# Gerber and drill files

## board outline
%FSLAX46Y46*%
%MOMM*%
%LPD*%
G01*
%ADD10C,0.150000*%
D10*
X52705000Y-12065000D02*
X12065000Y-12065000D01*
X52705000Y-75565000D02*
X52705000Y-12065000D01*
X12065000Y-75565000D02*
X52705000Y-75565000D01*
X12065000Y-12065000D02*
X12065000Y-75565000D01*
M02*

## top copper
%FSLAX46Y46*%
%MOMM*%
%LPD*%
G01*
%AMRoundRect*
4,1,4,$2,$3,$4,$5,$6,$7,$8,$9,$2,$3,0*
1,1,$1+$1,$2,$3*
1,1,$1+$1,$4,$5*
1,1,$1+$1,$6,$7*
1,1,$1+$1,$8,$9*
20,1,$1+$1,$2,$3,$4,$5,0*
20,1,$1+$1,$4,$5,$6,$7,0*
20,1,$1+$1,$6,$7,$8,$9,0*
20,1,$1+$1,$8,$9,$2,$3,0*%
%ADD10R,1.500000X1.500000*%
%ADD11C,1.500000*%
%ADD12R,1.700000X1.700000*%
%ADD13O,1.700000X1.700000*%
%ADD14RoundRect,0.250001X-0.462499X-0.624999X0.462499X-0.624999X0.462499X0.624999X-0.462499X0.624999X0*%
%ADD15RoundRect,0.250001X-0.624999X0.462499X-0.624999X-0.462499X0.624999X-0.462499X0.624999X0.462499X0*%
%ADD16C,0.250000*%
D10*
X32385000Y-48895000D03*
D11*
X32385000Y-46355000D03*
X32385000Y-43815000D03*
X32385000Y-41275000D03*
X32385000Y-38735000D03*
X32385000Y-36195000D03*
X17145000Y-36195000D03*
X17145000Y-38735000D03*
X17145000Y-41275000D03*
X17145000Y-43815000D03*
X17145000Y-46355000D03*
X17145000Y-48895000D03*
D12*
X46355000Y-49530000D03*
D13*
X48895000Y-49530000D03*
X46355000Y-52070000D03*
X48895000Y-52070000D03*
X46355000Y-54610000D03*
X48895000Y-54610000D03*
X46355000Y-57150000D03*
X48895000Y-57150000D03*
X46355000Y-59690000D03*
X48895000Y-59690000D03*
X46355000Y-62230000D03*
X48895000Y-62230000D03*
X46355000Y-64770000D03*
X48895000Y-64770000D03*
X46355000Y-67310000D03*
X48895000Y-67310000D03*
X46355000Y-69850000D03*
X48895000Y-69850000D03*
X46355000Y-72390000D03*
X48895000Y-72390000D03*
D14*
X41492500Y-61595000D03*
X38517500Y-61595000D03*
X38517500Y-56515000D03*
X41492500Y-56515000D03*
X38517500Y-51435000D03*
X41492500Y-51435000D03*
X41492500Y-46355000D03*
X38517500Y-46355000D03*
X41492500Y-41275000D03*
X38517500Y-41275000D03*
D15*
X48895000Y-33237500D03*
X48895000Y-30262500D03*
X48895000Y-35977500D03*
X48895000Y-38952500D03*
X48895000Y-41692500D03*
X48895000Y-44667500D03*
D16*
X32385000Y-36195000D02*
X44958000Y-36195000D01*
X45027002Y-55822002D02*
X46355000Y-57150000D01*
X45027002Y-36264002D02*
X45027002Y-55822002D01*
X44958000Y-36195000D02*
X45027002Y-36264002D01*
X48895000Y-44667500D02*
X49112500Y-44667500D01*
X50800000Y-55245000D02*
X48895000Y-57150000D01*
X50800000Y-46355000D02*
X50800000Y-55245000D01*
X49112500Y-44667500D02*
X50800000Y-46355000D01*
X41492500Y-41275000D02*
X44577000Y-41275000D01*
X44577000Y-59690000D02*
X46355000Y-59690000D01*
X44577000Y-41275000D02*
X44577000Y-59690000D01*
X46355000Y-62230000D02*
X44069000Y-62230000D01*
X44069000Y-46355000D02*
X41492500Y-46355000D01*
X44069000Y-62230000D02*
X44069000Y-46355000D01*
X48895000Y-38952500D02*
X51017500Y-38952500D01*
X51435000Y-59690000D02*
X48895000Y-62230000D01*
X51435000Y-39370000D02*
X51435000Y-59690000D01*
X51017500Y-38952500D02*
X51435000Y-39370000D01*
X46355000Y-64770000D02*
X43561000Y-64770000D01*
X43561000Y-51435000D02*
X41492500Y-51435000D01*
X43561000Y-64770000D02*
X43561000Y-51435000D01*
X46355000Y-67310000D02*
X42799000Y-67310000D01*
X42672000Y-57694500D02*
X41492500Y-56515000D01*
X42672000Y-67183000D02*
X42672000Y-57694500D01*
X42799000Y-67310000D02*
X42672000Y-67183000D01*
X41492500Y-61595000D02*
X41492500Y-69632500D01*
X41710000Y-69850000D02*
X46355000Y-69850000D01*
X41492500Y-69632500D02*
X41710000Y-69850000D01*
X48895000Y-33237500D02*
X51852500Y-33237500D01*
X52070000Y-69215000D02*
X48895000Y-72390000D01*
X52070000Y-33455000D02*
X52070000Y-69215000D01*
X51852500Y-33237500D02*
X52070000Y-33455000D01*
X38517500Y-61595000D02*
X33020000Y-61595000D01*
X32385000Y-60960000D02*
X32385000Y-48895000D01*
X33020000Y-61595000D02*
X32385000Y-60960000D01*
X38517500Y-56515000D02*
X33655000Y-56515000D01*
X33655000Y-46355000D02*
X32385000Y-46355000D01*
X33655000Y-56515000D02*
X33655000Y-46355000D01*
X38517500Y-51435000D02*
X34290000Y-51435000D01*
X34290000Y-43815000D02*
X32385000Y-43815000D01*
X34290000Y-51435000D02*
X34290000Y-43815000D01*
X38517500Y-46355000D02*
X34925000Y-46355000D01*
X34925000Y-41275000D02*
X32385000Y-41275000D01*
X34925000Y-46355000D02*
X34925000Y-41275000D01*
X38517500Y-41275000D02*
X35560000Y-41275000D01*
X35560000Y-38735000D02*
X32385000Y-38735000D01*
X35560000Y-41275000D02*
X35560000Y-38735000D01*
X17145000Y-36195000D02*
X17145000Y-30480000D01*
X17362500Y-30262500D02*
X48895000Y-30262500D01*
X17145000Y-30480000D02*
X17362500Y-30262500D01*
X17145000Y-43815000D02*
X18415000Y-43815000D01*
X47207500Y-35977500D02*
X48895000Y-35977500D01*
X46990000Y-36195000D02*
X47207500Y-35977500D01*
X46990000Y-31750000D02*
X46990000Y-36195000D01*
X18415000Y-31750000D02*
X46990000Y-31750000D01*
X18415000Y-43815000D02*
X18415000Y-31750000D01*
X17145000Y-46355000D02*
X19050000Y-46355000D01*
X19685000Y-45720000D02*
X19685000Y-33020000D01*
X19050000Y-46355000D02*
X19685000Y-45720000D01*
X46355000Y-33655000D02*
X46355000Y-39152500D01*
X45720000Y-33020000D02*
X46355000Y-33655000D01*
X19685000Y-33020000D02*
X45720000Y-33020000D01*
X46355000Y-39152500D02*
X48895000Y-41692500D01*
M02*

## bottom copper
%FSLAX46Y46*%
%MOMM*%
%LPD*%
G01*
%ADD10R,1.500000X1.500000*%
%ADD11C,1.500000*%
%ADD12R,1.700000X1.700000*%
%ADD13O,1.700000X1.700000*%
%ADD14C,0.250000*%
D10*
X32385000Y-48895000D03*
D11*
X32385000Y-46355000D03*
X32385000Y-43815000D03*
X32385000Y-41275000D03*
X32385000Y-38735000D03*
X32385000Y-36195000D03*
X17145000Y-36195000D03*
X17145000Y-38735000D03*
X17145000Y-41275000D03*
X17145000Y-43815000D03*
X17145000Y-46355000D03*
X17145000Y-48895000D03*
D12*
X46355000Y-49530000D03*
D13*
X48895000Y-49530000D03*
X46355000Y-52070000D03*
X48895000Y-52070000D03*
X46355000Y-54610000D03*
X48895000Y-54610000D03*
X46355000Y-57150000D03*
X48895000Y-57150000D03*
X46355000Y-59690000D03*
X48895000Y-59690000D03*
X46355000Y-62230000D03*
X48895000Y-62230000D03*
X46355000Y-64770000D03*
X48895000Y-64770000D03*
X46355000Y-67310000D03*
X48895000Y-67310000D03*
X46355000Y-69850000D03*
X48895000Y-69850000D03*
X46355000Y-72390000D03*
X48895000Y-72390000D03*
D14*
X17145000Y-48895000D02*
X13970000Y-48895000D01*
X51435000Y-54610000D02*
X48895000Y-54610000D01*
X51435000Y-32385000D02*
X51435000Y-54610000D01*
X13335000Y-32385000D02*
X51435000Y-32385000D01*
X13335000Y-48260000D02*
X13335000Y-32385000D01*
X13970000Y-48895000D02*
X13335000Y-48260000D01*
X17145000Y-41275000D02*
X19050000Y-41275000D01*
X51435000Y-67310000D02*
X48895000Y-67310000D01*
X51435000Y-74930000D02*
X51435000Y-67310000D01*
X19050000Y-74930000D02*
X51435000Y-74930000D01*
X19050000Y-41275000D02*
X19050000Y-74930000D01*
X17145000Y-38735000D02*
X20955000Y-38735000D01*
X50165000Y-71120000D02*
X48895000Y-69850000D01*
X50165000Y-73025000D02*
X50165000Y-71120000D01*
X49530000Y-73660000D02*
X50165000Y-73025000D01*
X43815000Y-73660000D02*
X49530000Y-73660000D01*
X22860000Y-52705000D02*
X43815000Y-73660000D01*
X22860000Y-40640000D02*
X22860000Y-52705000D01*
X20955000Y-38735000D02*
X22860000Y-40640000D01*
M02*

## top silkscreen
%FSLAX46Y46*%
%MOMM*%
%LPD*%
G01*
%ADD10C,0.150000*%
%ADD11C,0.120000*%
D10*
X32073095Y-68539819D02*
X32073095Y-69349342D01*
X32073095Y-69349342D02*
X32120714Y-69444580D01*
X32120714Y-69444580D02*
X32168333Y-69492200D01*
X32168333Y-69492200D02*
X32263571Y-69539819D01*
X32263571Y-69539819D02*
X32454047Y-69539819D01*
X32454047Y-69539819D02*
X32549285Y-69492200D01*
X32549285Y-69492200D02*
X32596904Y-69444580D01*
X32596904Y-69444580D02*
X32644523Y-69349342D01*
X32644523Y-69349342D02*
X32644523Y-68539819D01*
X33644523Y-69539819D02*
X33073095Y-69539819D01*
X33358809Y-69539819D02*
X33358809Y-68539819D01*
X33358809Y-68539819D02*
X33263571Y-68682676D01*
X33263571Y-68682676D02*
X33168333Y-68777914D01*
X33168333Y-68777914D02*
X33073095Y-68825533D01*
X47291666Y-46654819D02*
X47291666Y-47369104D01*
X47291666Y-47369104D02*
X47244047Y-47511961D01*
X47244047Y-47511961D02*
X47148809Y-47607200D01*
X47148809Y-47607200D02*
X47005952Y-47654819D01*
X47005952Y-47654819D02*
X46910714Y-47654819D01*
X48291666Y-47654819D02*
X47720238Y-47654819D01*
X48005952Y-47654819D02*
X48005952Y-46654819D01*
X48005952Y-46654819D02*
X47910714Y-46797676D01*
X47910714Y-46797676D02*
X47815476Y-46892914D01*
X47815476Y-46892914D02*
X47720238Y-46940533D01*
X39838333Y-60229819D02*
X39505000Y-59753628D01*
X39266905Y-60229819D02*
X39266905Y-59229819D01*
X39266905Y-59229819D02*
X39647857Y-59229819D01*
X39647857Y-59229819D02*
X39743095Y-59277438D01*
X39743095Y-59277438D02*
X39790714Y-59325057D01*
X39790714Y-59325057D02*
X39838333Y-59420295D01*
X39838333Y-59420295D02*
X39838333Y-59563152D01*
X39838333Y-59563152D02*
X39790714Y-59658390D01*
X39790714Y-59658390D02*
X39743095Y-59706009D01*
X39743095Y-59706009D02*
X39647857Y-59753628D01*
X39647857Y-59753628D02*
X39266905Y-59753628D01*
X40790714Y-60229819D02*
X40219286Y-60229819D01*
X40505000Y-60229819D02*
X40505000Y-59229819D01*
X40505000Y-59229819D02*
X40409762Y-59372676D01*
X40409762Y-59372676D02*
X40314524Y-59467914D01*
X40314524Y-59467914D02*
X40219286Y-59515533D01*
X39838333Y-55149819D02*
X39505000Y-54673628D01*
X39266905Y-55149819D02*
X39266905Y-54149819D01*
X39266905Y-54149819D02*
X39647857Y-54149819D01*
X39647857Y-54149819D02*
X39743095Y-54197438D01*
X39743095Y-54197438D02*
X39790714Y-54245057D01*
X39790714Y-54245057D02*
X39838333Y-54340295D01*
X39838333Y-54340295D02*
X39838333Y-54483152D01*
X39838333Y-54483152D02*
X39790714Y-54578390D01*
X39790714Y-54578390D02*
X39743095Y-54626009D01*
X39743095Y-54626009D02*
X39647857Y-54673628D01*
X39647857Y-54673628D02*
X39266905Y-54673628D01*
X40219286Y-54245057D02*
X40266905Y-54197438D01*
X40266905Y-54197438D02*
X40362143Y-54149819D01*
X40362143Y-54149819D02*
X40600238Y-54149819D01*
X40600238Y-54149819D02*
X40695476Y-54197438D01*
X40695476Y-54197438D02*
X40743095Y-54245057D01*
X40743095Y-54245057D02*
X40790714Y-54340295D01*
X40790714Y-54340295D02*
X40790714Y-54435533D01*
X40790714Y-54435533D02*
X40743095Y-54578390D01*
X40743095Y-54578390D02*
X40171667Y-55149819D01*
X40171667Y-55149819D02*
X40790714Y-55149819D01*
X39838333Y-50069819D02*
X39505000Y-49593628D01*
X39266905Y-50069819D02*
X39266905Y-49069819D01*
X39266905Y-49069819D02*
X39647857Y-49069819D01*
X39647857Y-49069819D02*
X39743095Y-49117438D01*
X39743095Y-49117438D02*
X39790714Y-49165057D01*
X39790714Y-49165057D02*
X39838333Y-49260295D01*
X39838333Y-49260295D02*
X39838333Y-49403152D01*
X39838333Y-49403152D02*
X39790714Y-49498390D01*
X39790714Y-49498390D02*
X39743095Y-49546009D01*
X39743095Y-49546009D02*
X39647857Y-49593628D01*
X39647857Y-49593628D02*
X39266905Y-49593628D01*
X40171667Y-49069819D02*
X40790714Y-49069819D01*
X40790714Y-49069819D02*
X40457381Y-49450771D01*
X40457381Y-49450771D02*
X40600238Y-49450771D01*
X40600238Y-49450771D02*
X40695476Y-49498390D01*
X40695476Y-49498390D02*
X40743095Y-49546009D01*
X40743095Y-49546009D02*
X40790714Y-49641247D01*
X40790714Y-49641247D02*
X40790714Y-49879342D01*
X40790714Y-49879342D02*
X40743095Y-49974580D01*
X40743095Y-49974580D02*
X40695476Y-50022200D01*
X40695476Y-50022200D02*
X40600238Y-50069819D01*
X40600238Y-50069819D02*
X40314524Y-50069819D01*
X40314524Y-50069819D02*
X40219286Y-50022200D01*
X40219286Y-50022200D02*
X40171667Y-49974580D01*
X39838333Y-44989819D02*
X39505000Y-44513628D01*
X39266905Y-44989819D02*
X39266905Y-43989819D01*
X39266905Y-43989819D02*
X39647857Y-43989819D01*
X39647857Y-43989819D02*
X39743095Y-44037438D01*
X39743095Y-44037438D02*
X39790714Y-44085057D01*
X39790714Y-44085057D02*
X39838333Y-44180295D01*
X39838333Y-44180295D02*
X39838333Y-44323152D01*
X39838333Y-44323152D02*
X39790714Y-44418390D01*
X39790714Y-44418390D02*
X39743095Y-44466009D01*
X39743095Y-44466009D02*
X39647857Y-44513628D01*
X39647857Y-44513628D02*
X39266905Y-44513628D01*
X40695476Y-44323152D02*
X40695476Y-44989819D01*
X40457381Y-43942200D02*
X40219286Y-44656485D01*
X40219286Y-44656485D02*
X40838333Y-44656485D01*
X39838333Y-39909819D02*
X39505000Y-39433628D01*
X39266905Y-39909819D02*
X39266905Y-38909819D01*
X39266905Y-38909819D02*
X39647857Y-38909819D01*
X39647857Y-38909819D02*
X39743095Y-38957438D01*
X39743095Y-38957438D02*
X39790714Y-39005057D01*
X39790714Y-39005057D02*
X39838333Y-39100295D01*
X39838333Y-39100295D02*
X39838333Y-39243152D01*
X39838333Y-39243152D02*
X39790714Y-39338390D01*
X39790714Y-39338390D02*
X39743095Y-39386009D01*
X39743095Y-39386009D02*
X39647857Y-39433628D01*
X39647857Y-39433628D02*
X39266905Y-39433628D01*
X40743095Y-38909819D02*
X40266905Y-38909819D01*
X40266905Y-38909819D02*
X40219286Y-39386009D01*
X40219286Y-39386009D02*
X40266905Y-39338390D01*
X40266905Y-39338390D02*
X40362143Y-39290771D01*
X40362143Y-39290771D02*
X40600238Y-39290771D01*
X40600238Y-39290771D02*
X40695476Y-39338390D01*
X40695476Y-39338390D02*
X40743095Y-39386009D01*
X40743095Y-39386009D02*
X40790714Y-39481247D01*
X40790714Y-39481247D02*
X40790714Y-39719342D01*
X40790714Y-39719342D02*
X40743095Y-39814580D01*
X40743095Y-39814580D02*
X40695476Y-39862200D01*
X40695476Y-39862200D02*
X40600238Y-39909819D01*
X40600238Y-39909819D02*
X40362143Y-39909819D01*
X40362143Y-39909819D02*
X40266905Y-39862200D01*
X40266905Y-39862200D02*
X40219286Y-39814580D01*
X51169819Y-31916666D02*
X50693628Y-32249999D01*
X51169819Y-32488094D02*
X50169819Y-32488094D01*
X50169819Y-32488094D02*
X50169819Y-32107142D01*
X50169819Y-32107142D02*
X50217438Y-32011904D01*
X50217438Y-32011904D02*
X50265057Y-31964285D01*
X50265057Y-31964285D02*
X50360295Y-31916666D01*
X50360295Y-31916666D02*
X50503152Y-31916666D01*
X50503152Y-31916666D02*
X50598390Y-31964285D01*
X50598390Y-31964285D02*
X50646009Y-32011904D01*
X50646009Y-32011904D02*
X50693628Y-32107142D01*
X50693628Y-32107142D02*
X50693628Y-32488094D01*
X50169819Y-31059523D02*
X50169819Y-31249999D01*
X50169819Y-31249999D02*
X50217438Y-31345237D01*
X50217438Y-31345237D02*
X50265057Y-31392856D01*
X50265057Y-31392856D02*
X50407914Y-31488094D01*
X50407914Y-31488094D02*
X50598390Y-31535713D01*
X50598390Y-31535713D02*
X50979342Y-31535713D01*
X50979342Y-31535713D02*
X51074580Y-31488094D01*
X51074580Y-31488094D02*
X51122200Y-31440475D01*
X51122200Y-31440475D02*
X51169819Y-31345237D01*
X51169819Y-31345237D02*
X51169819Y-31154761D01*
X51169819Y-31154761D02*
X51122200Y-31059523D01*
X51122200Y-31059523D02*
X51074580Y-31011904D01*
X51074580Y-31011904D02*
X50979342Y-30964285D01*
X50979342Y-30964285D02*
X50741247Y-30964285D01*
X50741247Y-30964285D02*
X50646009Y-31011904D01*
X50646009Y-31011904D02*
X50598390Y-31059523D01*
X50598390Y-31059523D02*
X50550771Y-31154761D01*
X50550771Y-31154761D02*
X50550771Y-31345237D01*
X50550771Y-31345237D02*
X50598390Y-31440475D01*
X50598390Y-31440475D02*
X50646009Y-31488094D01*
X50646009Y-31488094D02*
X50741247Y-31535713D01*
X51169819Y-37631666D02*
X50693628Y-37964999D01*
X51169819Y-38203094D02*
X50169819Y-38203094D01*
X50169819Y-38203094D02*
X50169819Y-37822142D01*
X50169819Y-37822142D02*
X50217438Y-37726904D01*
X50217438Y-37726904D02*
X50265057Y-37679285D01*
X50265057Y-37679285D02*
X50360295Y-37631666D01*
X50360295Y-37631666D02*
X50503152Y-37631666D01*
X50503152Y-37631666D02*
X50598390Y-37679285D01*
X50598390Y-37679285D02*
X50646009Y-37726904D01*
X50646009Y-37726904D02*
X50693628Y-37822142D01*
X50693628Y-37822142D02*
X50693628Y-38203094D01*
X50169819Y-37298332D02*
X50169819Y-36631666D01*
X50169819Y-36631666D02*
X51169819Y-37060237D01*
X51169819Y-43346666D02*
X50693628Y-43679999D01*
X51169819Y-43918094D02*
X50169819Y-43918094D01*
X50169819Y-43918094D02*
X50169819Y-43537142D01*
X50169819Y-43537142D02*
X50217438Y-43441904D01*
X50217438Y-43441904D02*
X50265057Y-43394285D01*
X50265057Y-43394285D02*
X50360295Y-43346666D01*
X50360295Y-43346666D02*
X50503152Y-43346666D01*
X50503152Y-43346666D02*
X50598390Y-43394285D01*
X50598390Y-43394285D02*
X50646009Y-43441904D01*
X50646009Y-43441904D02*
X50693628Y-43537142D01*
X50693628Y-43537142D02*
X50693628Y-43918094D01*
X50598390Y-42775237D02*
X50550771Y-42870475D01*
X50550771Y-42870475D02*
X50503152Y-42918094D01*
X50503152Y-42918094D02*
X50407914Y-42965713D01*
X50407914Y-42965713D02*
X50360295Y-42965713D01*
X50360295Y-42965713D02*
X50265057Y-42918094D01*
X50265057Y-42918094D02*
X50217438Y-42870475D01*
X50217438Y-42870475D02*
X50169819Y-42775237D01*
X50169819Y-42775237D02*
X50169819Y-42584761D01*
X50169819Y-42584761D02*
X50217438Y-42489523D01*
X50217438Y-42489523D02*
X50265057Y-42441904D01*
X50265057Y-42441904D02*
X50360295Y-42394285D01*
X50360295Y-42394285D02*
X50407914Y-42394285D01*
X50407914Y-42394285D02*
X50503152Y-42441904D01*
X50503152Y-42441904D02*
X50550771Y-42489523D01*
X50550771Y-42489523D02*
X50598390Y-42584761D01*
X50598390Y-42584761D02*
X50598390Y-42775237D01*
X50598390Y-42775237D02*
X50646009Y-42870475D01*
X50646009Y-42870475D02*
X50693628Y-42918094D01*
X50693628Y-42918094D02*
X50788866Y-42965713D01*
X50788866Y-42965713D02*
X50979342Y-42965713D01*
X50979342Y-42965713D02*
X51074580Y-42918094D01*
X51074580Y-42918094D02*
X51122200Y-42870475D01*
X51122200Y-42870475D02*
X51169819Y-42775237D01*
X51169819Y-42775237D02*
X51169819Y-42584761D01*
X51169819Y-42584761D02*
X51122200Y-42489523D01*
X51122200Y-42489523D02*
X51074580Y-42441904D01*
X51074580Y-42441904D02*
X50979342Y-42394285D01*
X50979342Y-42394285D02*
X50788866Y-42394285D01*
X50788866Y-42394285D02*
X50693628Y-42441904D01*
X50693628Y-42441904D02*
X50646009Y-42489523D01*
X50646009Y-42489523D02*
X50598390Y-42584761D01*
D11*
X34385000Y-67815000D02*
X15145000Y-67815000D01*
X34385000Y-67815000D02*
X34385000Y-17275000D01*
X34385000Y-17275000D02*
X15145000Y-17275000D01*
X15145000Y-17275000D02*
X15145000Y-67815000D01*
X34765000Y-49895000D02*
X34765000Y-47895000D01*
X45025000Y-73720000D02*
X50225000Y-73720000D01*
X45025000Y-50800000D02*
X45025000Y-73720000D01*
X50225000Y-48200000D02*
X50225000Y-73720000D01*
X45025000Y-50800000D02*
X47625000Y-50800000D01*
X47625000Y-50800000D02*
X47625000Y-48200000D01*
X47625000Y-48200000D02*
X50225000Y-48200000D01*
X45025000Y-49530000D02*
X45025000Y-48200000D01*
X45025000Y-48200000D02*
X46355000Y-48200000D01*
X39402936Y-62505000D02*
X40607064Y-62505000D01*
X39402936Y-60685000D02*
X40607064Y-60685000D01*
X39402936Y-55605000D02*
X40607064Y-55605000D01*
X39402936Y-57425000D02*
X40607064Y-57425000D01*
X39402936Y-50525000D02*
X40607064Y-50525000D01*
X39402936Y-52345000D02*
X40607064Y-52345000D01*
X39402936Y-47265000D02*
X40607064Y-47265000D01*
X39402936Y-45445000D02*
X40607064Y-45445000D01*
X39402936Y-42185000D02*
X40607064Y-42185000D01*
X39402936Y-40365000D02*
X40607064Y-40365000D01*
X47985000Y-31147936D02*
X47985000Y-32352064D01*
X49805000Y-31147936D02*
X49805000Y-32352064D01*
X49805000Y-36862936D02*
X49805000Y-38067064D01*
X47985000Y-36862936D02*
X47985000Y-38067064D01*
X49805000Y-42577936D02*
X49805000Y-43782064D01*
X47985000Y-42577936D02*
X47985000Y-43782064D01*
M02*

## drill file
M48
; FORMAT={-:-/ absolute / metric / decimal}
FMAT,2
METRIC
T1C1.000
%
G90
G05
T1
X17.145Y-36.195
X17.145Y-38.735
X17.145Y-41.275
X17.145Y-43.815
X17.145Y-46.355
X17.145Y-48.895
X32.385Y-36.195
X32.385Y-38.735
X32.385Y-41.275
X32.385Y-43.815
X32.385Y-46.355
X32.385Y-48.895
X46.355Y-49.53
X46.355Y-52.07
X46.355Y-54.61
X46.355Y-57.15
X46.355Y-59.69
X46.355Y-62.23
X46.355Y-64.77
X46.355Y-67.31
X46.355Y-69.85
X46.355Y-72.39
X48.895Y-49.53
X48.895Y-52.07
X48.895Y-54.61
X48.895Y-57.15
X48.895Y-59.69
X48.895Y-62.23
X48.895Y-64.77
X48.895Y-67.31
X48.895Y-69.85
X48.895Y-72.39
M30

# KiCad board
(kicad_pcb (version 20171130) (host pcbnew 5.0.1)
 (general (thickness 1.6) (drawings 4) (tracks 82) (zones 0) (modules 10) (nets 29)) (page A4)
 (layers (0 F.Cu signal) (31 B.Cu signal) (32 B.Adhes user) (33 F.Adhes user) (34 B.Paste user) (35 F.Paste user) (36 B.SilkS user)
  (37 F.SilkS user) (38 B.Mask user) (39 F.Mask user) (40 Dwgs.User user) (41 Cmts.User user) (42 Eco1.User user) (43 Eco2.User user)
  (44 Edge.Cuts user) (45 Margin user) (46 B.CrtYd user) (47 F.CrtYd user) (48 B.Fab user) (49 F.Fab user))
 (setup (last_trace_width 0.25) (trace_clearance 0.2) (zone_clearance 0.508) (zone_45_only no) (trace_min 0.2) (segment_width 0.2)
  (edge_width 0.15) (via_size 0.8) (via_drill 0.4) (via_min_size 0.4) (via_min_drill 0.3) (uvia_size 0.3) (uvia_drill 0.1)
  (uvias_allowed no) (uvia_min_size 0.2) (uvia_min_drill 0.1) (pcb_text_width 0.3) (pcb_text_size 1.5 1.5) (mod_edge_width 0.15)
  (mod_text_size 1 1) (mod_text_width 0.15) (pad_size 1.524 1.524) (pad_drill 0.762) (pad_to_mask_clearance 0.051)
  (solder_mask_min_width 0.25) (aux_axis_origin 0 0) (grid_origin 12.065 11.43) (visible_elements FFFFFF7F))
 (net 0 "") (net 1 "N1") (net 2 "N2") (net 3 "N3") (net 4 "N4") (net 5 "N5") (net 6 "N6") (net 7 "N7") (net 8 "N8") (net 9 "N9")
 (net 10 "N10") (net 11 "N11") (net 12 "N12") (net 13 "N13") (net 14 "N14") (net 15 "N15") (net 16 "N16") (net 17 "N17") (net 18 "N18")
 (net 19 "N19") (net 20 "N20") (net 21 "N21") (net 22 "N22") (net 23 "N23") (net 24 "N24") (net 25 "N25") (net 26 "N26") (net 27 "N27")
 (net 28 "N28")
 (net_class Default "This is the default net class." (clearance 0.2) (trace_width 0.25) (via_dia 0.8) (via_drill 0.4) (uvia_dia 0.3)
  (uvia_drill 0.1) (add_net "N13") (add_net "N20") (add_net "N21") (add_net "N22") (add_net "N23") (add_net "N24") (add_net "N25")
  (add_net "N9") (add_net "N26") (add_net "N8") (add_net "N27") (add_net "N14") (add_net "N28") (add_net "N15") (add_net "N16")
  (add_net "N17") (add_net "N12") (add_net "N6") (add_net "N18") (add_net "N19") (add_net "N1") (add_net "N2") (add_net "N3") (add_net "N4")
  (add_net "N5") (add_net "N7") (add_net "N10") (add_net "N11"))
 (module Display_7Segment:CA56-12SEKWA (layer F.Cu) (at 32.385 48.895 180)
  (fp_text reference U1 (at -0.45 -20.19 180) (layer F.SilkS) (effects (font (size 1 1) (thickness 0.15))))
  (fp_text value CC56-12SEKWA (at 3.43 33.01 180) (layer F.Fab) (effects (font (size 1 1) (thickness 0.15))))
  (fp_line (start -2 -18.92) (end 17.24 -18.92) (layer F.SilkS) (width 0.12))
  (fp_line (start -2 -18.92) (end -2 31.62) (layer F.SilkS) (width 0.12))
  (fp_line (start -2 31.62) (end 17.24 31.62) (layer F.SilkS) (width 0.12))
  (fp_line (start 17.24 31.62) (end 17.24 -18.92) (layer F.SilkS) (width 0.12))
  (fp_line (start -2.38 -1) (end -2.38 1) (layer F.SilkS) (width 0.12))
  (pad 1 thru_hole rect (at 0 0 180) (size 1.5 1.5) (drill 1) (layers *.Cu *.Mask) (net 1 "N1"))
  (pad 2 thru_hole circle (at 0 2.54 180) (size 1.5 1.5) (drill 1) (layers *.Cu *.Mask) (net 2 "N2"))
  (pad 3 thru_hole circle (at 0 5.08 180) (size 1.5 1.5) (drill 1) (layers *.Cu *.Mask) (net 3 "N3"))
  (pad 4 thru_hole circle (at 0 7.62 180) (size 1.5 1.5) (drill 1) (layers *.Cu *.Mask) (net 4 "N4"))
  (pad 5 thru_hole circle (at 0 10.16 180) (size 1.5 1.5) (drill 1) (layers *.Cu *.Mask) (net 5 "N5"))
  (pad 6 thru_hole circle (at 0 12.7 180) (size 1.5 1.5) (drill 1) (layers *.Cu *.Mask) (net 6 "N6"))
  (pad 7 thru_hole circle (at 15.24 12.7 180) (size 1.5 1.5) (drill 1) (layers *.Cu *.Mask) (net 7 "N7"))
  (pad 8 thru_hole circle (at 15.24 10.16 180) (size 1.5 1.5) (drill 1) (layers *.Cu *.Mask) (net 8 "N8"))
  (pad 9 thru_hole circle (at 15.24 7.62 180) (size 1.5 1.5) (drill 1) (layers *.Cu *.Mask) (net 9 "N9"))
  (pad 10 thru_hole circle (at 15.24 5.08 180) (size 1.5 1.5) (drill 1) (layers *.Cu *.Mask) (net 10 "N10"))
  (pad 11 thru_hole circle (at 15.24 2.54 180) (size 1.5 1.5) (drill 1) (layers *.Cu *.Mask) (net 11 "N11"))
  (pad 12 thru_hole circle (at 15.24 0 180) (size 1.5 1.5) (drill 1) (layers *.Cu *.Mask) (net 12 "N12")))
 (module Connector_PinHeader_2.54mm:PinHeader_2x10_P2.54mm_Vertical (layer F.Cu) (at 46.355 49.53)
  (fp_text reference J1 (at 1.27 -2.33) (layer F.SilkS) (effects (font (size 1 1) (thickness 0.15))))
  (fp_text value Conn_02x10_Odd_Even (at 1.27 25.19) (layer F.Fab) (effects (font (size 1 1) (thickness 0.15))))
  (fp_line (start -1.33 24.19) (end 3.87 24.19) (layer F.SilkS) (width 0.12))
  (fp_line (start -1.33 1.27) (end -1.33 24.19) (layer F.SilkS) (width 0.12))
  (fp_line (start 3.87 -1.33) (end 3.87 24.19) (layer F.SilkS) (width 0.12))
  (fp_line (start -1.33 1.27) (end 1.27 1.27) (layer F.SilkS) (width 0.12))
  (fp_line (start 1.27 1.27) (end 1.27 -1.33) (layer F.SilkS) (width 0.12))
  (fp_line (start 1.27 -1.33) (end 3.87 -1.33) (layer F.SilkS) (width 0.12))
  (fp_line (start -1.33 0) (end -1.33 -1.33) (layer F.SilkS) (width 0.12))
  (fp_line (start -1.33 -1.33) (end 0 -1.33) (layer F.SilkS) (width 0.12))
  (pad 1 thru_hole rect (at 0 0) (size 1.7 1.7) (drill 1) (layers *.Cu *.Mask) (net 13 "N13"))
  (pad 2 thru_hole oval (at 2.54 0) (size 1.7 1.7) (drill 1) (layers *.Cu *.Mask) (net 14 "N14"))
  (pad 3 thru_hole oval (at 0 2.54) (size 1.7 1.7) (drill 1) (layers *.Cu *.Mask) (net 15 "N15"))
  (pad 4 thru_hole oval (at 2.54 2.54) (size 1.7 1.7) (drill 1) (layers *.Cu *.Mask) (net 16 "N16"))
  (pad 5 thru_hole oval (at 0 5.08) (size 1.7 1.7) (drill 1) (layers *.Cu *.Mask) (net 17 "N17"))
  (pad 6 thru_hole oval (at 2.54 5.08) (size 1.7 1.7) (drill 1) (layers *.Cu *.Mask) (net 12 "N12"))
  (pad 7 thru_hole oval (at 0 7.62) (size 1.7 1.7) (drill 1) (layers *.Cu *.Mask) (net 6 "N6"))
  (pad 8 thru_hole oval (at 2.54 7.62) (size 1.7 1.7) (drill 1) (layers *.Cu *.Mask) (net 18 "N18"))
  (pad 9 thru_hole oval (at 0 10.16) (size 1.7 1.7) (drill 1) (layers *.Cu *.Mask) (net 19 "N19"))
  (pad 10 thru_hole oval (at 2.54 10.16) (size 1.7 1.7) (drill 1) (layers *.Cu *.Mask) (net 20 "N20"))
  (pad 11 thru_hole oval (at 0 12.7) (size 1.7 1.7) (drill 1) (layers *.Cu *.Mask) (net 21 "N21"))
  (pad 12 thru_hole oval (at 2.54 12.7) (size 1.7 1.7) (drill 1) (layers *.Cu *.Mask) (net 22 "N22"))
  (pad 13 thru_hole oval (at 0 15.24) (size 1.7 1.7) (drill 1) (layers *.Cu *.Mask) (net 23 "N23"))
  (pad 14 thru_hole oval (at 2.54 15.24) (size 1.7 1.7) (drill 1) (layers *.Cu *.Mask) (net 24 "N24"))
  (pad 15 thru_hole oval (at 0 17.78) (size 1.7 1.7) (drill 1) (layers *.Cu *.Mask) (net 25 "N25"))
  (pad 16 thru_hole oval (at 2.54 17.78) (size 1.7 1.7) (drill 1) (layers *.Cu *.Mask) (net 9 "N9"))
  (pad 17 thru_hole oval (at 0 20.32) (size 1.7 1.7) (drill 1) (layers *.Cu *.Mask) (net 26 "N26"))
  (pad 18 thru_hole oval (at 2.54 20.32) (size 1.7 1.7) (drill 1) (layers *.Cu *.Mask) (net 8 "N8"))
  (pad 19 thru_hole oval (at 0 22.86) (size 1.7 1.7) (drill 1) (layers *.Cu *.Mask) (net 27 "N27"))
  (pad 20 thru_hole oval (at 2.54 22.86) (size 1.7 1.7) (drill 1) (layers *.Cu *.Mask) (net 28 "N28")))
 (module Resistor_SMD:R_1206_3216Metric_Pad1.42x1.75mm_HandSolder (layer F.Cu) (at 40.005 61.595)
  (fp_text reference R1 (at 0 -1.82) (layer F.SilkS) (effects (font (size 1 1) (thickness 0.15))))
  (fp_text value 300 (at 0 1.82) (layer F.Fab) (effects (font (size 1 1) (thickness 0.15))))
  (fp_line (start -0.602064 0.91) (end 0.602064 0.91) (layer F.SilkS) (width 0.12))
  (fp_line (start -0.602064 -0.91) (end 0.602064 -0.91) (layer F.SilkS) (width 0.12))
  (pad 2 smd roundrect (at 1.4875 0) (size 1.425 1.75) (layers F.Cu F.Paste F.Mask) (roundrect_rratio 0.175439) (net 26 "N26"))
  (pad 1 smd roundrect (at -1.4875 0) (size 1.425 1.75) (layers F.Cu F.Paste F.Mask) (roundrect_rratio 0.175439) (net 1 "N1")))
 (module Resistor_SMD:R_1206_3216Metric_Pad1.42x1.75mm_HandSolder (layer F.Cu) (at 40.005 56.515)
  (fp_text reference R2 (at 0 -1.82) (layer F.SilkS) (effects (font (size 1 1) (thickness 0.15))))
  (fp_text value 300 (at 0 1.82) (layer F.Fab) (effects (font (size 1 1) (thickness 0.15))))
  (fp_line (start -0.602064 -0.91) (end 0.602064 -0.91) (layer F.SilkS) (width 0.12))
  (fp_line (start -0.602064 0.91) (end 0.602064 0.91) (layer F.SilkS) (width 0.12))
  (pad 1 smd roundrect (at -1.4875 0) (size 1.425 1.75) (layers F.Cu F.Paste F.Mask) (roundrect_rratio 0.175439) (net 2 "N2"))
  (pad 2 smd roundrect (at 1.4875 0) (size 1.425 1.75) (layers F.Cu F.Paste F.Mask) (roundrect_rratio 0.175439) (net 25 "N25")))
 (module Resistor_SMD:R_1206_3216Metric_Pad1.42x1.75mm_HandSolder (layer F.Cu) (at 40.005 51.435)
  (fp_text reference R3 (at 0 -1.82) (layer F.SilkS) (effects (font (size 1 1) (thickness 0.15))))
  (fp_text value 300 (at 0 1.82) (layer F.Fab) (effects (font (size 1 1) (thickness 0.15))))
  (fp_line (start -0.602064 -0.91) (end 0.602064 -0.91) (layer F.SilkS) (width 0.12))
  (fp_line (start -0.602064 0.91) (end 0.602064 0.91) (layer F.SilkS) (width 0.12))
  (pad 1 smd roundrect (at -1.4875 0) (size 1.425 1.75) (layers F.Cu F.Paste F.Mask) (roundrect_rratio 0.175439) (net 3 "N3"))
  (pad 2 smd roundrect (at 1.4875 0) (size 1.425 1.75) (layers F.Cu F.Paste F.Mask) (roundrect_rratio 0.175439) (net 23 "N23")))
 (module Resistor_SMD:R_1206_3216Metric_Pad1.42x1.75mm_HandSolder (layer F.Cu) (at 40.005 46.355)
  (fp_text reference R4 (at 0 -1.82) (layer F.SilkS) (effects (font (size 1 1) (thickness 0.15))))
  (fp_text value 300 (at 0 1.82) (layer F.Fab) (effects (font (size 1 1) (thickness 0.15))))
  (fp_line (start -0.602064 0.91) (end 0.602064 0.91) (layer F.SilkS) (width 0.12))
  (fp_line (start -0.602064 -0.91) (end 0.602064 -0.91) (layer F.SilkS) (width 0.12))
  (pad 2 smd roundrect (at 1.4875 0) (size 1.425 1.75) (layers F.Cu F.Paste F.Mask) (roundrect_rratio 0.175439) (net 21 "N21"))
  (pad 1 smd roundrect (at -1.4875 0) (size 1.425 1.75) (layers F.Cu F.Paste F.Mask) (roundrect_rratio 0.175439) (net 4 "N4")))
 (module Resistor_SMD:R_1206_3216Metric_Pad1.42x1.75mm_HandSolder (layer F.Cu) (at 40.005 41.275)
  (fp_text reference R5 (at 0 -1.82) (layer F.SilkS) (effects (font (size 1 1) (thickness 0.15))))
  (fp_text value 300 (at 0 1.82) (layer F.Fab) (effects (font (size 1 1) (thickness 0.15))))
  (fp_line (start -0.602064 0.91) (end 0.602064 0.91) (layer F.SilkS) (width 0.12))
  (fp_line (start -0.602064 -0.91) (end 0.602064 -0.91) (layer F.SilkS) (width 0.12))
  (pad 2 smd roundrect (at 1.4875 0) (size 1.425 1.75) (layers F.Cu F.Paste F.Mask) (roundrect_rratio 0.175439) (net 19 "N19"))
  (pad 1 smd roundrect (at -1.4875 0) (size 1.425 1.75) (layers F.Cu F.Paste F.Mask) (roundrect_rratio 0.175439) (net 5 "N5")))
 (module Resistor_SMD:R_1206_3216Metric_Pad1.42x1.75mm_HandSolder (layer F.Cu) (at 48.895 31.75 270)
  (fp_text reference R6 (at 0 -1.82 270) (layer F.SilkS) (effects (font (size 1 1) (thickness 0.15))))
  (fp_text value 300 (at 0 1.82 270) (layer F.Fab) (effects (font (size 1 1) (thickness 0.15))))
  (fp_line (start -0.602064 0.91) (end 0.602064 0.91) (layer F.SilkS) (width 0.12))
  (fp_line (start -0.602064 -0.91) (end 0.602064 -0.91) (layer F.SilkS) (width 0.12))
  (pad 2 smd roundrect (at 1.4875 0 270) (size 1.425 1.75) (layers F.Cu F.Paste F.Mask) (roundrect_rratio 0.175439) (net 28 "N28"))
  (pad 1 smd roundrect (at -1.4875 0 270) (size 1.425 1.75) (layers F.Cu F.Paste F.Mask) (roundrect_rratio 0.175439) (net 7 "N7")))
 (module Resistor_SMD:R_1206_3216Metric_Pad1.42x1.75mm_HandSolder (layer F.Cu) (at 48.895 37.465 270)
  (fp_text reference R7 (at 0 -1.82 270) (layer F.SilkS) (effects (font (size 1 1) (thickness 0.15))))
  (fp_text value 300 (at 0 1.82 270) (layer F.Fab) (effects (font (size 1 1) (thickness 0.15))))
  (fp_line (start -0.602064 -0.91) (end 0.602064 -0.91) (layer F.SilkS) (width 0.12))
  (fp_line (start -0.602064 0.91) (end 0.602064 0.91) (layer F.SilkS) (width 0.12))
  (pad 1 smd roundrect (at -1.4875 0 270) (size 1.425 1.75) (layers F.Cu F.Paste F.Mask) (roundrect_rratio 0.175439) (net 10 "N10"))
  (pad 2 smd roundrect (at 1.4875 0 270) (size 1.425 1.75) (layers F.Cu F.Paste F.Mask) (roundrect_rratio 0.175439) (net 22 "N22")))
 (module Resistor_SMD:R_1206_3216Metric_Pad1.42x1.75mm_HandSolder (layer F.Cu) (at 48.895 43.18 270)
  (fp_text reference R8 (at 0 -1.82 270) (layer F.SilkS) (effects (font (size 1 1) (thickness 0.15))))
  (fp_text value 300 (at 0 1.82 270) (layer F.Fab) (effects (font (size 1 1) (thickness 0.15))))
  (fp_line (start -0.602064 -0.91) (end 0.602064 -0.91) (layer F.SilkS) (width 0.12))
  (fp_line (start -0.602064 0.91) (end 0.602064 0.91) (layer F.SilkS) (width 0.12))
  (pad 1 smd roundrect (at -1.4875 0 270) (size 1.425 1.75) (layers F.Cu F.Paste F.Mask) (roundrect_rratio 0.175439) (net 11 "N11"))
  (pad 2 smd roundrect (at 1.4875 0 270) (size 1.425 1.75) (layers F.Cu F.Paste F.Mask) (roundrect_rratio 0.175439) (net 18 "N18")))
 (gr_line (start 52.705 12.065) (end 12.065 12.065) (angle 90) (layer Edge.Cuts) (width 0.15))
 (gr_line (start 52.705 75.565) (end 52.705 12.065) (angle 90) (layer Edge.Cuts) (width 0.15))
 (gr_line (start 12.065 75.565) (end 52.705 75.565) (angle 90) (layer Edge.Cuts) (width 0.15))
 (gr_line (start 12.065 12.065) (end 12.065 75.565) (angle 90) (layer Edge.Cuts) (width 0.15))
 (segment (start 17.145 48.895) (end 13.97 48.895) (width 0.25) (layer B.Cu) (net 12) (status 400000))
 (segment (start 51.435 54.61) (end 48.895 54.61) (width 0.25) (layer B.Cu) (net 12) (status 800000))
 (segment (start 51.435 32.385) (end 51.435 54.61) (width 0.25) (layer B.Cu) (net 12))
 (segment (start 13.335 32.385) (end 51.435 32.385) (width 0.25) (layer B.Cu) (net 12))
 (segment (start 13.335 48.26) (end 13.335 32.385) (width 0.25) (layer B.Cu) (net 12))
 (segment (start 13.97 48.895) (end 13.335 48.26) (width 0.25) (layer B.Cu) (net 12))
 (segment (start 32.385 36.195) (end 44.958 36.195) (width 0.25) (layer F.Cu) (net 6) (status 400000))
 (segment (start 45.027002 55.822002) (end 46.355 57.15) (width 0.25) (layer F.Cu) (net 6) (status 800000))
 (segment (start 45.027002 36.264002) (end 45.027002 55.822002) (width 0.25) (layer F.Cu) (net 6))
 (segment (start 44.958 36.195) (end 45.027002 36.264002) (width 0.25) (layer F.Cu) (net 6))
 (segment (start 48.895 44.6675) (end 49.1125 44.6675) (width 0.25) (layer F.Cu) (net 18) (status C00000))
 (segment (start 50.8 55.245) (end 48.895 57.15) (width 0.25) (layer F.Cu) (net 18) (status 800000))
 (segment (start 50.8 46.355) (end 50.8 55.245) (width 0.25) (layer F.Cu) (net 18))
 (segment (start 49.1125 44.6675) (end 50.8 46.355) (width 0.25) (layer F.Cu) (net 18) (status 400000))
 (segment (start 41.4925 41.275) (end 44.577 41.275) (width 0.25) (layer F.Cu) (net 19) (status 400000))
 (segment (start 44.577 59.69) (end 46.355 59.69) (width 0.25) (layer F.Cu) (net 19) (status 800000))
 (segment (start 44.577 41.275) (end 44.577 59.69) (width 0.25) (layer F.Cu) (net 19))
 (segment (start 46.355 62.23) (end 44.069 62.23) (width 0.25) (layer F.Cu) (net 21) (status 400000))
 (segment (start 44.069 46.355) (end 41.4925 46.355) (width 0.25) (layer F.Cu) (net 21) (status 800000))
 (segment (start 44.069 62.23) (end 44.069 46.355) (width 0.25) (layer F.Cu) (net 21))
 (segment (start 48.895 38.9525) (end 51.0175 38.9525) (width 0.25) (layer F.Cu) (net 22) (status 400000))
 (segment (start 51.435 59.69) (end 48.895 62.23) (width 0.25) (layer F.Cu) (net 22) (status 800000))
 (segment (start 51.435 39.37) (end 51.435 59.69) (width 0.25) (layer F.Cu) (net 22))
 (segment (start 51.0175 38.9525) (end 51.435 39.37) (width 0.25) (layer F.Cu) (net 22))
 (segment (start 46.355 64.77) (end 43.561 64.77) (width 0.25) (layer F.Cu) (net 23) (status 400000))
 (segment (start 43.561 51.435) (end 41.4925 51.435) (width 0.25) (layer F.Cu) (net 23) (status 800000))
 (segment (start 43.561 64.77) (end 43.561 51.435) (width 0.25) (layer F.Cu) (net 23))
 (segment (start 46.355 67.31) (end 42.799 67.31) (width 0.25) (layer F.Cu) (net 25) (status 400000))
 (segment (start 42.672 57.6945) (end 41.4925 56.515) (width 0.25) (layer F.Cu) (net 25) (status 800000))
 (segment (start 42.672 67.183) (end 42.672 57.6945) (width 0.25) (layer F.Cu) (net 25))
 (segment (start 42.799 67.31) (end 42.672 67.183) (width 0.25) (layer F.Cu) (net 25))
 (segment (start 17.145 41.275) (end 19.05 41.275) (width 0.25) (layer B.Cu) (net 9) (status 400000))
 (segment (start 51.435 67.31) (end 48.895 67.31) (width 0.25) (layer B.Cu) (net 9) (status 800000))
 (segment (start 51.435 74.93) (end 51.435 67.31) (width 0.25) (layer B.Cu) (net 9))
 (segment (start 19.05 74.93) (end 51.435 74.93) (width 0.25) (layer B.Cu) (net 9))
 (segment (start 19.05 41.275) (end 19.05 74.93) (width 0.25) (layer B.Cu) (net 9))
 (segment (start 41.4925 61.595) (end 41.4925 69.6325) (width 0.25) (layer F.Cu) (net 26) (status 400000))
 (segment (start 41.71 69.85) (end 46.355 69.85) (width 0.25) (layer F.Cu) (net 26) (status 800000))
 (segment (start 41.4925 69.6325) (end 41.71 69.85) (width 0.25) (layer F.Cu) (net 26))
 (segment (start 17.145 38.735) (end 20.955 38.735) (width 0.25) (layer B.Cu) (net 8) (status 400000))
 (segment (start 50.165 71.12) (end 48.895 69.85) (width 0.25) (layer B.Cu) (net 8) (status 800000))
 (segment (start 50.165 73.025) (end 50.165 71.12) (width 0.25) (layer B.Cu) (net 8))
 (segment (start 49.53 73.66) (end 50.165 73.025) (width 0.25) (layer B.Cu) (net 8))
 (segment (start 43.815 73.66) (end 49.53 73.66) (width 0.25) (layer B.Cu) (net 8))
 (segment (start 22.86 52.705) (end 43.815 73.66) (width 0.25) (layer B.Cu) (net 8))
 (segment (start 22.86 40.64) (end 22.86 52.705) (width 0.25) (layer B.Cu) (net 8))
 (segment (start 20.955 38.735) (end 22.86 40.64) (width 0.25) (layer B.Cu) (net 8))
 (segment (start 48.895 33.2375) (end 51.8525 33.2375) (width 0.25) (layer F.Cu) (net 28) (status 400000))
 (segment (start 52.07 69.215) (end 48.895 72.39) (width 0.25) (layer F.Cu) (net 28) (status 800000))
 (segment (start 52.07 33.455) (end 52.07 69.215) (width 0.25) (layer F.Cu) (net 28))
 (segment (start 51.8525 33.2375) (end 52.07 33.455) (width 0.25) (layer F.Cu) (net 28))
 (segment (start 38.5175 61.595) (end 33.02 61.595) (width 0.25) (layer F.Cu) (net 1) (status 400000))
 (segment (start 32.385 60.96) (end 32.385 48.895) (width 0.25) (layer F.Cu) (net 1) (status 800000))
 (segment (start 33.02 61.595) (end 32.385 60.96) (width 0.25) (layer F.Cu) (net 1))
 (segment (start 38.5175 56.515) (end 33.655 56.515) (width 0.25) (layer F.Cu) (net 2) (status 400000))
 (segment (start 33.655 46.355) (end 32.385 46.355) (width 0.25) (layer F.Cu) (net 2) (status 800000))
 (segment (start 33.655 56.515) (end 33.655 46.355) (width 0.25) (layer F.Cu) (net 2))
 (segment (start 38.5175 51.435) (end 34.29 51.435) (width 0.25) (layer F.Cu) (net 3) (status 400000))
 (segment (start 34.29 43.815) (end 32.385 43.815) (width 0.25) (layer F.Cu) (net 3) (status 800000))
 (segment (start 34.29 51.435) (end 34.29 43.815) (width 0.25) (layer F.Cu) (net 3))
 (segment (start 38.5175 46.355) (end 34.925 46.355) (width 0.25) (layer F.Cu) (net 4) (status 400000))
 (segment (start 34.925 41.275) (end 32.385 41.275) (width 0.25) (layer F.Cu) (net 4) (status 800000))
 (segment (start 34.925 46.355) (end 34.925 41.275) (width 0.25) (layer F.Cu) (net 4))
 (segment (start 38.5175 41.275) (end 35.56 41.275) (width 0.25) (layer F.Cu) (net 5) (status 400000))
 (segment (start 35.56 38.735) (end 32.385 38.735) (width 0.25) (layer F.Cu) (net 5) (status 800000))
 (segment (start 35.56 41.275) (end 35.56 38.735) (width 0.25) (layer F.Cu) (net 5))
 (segment (start 17.145 36.195) (end 17.145 30.48) (width 0.25) (layer F.Cu) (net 7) (status 400000))
 (segment (start 17.3625 30.2625) (end 48.895 30.2625) (width 0.25) (layer F.Cu) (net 7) (status 800000))
 (segment (start 17.145 30.48) (end 17.3625 30.2625) (width 0.25) (layer F.Cu) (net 7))
 (segment (start 17.145 43.815) (end 18.415 43.815) (width 0.25) (layer F.Cu) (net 10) (status 400000))
 (segment (start 47.2075 35.9775) (end 48.895 35.9775) (width 0.25) (layer F.Cu) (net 10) (status 800000))
 (segment (start 46.99 36.195) (end 47.2075 35.9775) (width 0.25) (layer F.Cu) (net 10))
 (segment (start 46.99 31.75) (end 46.99 36.195) (width 0.25) (layer F.Cu) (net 10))
 (segment (start 18.415 31.75) (end 46.99 31.75) (width 0.25) (layer F.Cu) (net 10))
 (segment (start 18.415 43.815) (end 18.415 31.75) (width 0.25) (layer F.Cu) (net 10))
 (segment (start 17.145 46.355) (end 19.05 46.355) (width 0.25) (layer F.Cu) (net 11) (status 400000))
 (segment (start 19.685 45.72) (end 19.685 33.02) (width 0.25) (layer F.Cu) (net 11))
 (segment (start 19.05 46.355) (end 19.685 45.72) (width 0.25) (layer F.Cu) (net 11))
 (segment (start 46.355 33.655) (end 46.355 39.1525) (width 0.25) (layer F.Cu) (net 11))
 (segment (start 45.72 33.02) (end 46.355 33.655) (width 0.25) (layer F.Cu) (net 11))
 (segment (start 19.685 33.02) (end 45.72 33.02) (width 0.25) (layer F.Cu) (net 11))
 (segment (start 46.355 39.1525) (end 48.895 41.6925) (width 0.25) (layer F.Cu) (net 11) (status 800000)))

